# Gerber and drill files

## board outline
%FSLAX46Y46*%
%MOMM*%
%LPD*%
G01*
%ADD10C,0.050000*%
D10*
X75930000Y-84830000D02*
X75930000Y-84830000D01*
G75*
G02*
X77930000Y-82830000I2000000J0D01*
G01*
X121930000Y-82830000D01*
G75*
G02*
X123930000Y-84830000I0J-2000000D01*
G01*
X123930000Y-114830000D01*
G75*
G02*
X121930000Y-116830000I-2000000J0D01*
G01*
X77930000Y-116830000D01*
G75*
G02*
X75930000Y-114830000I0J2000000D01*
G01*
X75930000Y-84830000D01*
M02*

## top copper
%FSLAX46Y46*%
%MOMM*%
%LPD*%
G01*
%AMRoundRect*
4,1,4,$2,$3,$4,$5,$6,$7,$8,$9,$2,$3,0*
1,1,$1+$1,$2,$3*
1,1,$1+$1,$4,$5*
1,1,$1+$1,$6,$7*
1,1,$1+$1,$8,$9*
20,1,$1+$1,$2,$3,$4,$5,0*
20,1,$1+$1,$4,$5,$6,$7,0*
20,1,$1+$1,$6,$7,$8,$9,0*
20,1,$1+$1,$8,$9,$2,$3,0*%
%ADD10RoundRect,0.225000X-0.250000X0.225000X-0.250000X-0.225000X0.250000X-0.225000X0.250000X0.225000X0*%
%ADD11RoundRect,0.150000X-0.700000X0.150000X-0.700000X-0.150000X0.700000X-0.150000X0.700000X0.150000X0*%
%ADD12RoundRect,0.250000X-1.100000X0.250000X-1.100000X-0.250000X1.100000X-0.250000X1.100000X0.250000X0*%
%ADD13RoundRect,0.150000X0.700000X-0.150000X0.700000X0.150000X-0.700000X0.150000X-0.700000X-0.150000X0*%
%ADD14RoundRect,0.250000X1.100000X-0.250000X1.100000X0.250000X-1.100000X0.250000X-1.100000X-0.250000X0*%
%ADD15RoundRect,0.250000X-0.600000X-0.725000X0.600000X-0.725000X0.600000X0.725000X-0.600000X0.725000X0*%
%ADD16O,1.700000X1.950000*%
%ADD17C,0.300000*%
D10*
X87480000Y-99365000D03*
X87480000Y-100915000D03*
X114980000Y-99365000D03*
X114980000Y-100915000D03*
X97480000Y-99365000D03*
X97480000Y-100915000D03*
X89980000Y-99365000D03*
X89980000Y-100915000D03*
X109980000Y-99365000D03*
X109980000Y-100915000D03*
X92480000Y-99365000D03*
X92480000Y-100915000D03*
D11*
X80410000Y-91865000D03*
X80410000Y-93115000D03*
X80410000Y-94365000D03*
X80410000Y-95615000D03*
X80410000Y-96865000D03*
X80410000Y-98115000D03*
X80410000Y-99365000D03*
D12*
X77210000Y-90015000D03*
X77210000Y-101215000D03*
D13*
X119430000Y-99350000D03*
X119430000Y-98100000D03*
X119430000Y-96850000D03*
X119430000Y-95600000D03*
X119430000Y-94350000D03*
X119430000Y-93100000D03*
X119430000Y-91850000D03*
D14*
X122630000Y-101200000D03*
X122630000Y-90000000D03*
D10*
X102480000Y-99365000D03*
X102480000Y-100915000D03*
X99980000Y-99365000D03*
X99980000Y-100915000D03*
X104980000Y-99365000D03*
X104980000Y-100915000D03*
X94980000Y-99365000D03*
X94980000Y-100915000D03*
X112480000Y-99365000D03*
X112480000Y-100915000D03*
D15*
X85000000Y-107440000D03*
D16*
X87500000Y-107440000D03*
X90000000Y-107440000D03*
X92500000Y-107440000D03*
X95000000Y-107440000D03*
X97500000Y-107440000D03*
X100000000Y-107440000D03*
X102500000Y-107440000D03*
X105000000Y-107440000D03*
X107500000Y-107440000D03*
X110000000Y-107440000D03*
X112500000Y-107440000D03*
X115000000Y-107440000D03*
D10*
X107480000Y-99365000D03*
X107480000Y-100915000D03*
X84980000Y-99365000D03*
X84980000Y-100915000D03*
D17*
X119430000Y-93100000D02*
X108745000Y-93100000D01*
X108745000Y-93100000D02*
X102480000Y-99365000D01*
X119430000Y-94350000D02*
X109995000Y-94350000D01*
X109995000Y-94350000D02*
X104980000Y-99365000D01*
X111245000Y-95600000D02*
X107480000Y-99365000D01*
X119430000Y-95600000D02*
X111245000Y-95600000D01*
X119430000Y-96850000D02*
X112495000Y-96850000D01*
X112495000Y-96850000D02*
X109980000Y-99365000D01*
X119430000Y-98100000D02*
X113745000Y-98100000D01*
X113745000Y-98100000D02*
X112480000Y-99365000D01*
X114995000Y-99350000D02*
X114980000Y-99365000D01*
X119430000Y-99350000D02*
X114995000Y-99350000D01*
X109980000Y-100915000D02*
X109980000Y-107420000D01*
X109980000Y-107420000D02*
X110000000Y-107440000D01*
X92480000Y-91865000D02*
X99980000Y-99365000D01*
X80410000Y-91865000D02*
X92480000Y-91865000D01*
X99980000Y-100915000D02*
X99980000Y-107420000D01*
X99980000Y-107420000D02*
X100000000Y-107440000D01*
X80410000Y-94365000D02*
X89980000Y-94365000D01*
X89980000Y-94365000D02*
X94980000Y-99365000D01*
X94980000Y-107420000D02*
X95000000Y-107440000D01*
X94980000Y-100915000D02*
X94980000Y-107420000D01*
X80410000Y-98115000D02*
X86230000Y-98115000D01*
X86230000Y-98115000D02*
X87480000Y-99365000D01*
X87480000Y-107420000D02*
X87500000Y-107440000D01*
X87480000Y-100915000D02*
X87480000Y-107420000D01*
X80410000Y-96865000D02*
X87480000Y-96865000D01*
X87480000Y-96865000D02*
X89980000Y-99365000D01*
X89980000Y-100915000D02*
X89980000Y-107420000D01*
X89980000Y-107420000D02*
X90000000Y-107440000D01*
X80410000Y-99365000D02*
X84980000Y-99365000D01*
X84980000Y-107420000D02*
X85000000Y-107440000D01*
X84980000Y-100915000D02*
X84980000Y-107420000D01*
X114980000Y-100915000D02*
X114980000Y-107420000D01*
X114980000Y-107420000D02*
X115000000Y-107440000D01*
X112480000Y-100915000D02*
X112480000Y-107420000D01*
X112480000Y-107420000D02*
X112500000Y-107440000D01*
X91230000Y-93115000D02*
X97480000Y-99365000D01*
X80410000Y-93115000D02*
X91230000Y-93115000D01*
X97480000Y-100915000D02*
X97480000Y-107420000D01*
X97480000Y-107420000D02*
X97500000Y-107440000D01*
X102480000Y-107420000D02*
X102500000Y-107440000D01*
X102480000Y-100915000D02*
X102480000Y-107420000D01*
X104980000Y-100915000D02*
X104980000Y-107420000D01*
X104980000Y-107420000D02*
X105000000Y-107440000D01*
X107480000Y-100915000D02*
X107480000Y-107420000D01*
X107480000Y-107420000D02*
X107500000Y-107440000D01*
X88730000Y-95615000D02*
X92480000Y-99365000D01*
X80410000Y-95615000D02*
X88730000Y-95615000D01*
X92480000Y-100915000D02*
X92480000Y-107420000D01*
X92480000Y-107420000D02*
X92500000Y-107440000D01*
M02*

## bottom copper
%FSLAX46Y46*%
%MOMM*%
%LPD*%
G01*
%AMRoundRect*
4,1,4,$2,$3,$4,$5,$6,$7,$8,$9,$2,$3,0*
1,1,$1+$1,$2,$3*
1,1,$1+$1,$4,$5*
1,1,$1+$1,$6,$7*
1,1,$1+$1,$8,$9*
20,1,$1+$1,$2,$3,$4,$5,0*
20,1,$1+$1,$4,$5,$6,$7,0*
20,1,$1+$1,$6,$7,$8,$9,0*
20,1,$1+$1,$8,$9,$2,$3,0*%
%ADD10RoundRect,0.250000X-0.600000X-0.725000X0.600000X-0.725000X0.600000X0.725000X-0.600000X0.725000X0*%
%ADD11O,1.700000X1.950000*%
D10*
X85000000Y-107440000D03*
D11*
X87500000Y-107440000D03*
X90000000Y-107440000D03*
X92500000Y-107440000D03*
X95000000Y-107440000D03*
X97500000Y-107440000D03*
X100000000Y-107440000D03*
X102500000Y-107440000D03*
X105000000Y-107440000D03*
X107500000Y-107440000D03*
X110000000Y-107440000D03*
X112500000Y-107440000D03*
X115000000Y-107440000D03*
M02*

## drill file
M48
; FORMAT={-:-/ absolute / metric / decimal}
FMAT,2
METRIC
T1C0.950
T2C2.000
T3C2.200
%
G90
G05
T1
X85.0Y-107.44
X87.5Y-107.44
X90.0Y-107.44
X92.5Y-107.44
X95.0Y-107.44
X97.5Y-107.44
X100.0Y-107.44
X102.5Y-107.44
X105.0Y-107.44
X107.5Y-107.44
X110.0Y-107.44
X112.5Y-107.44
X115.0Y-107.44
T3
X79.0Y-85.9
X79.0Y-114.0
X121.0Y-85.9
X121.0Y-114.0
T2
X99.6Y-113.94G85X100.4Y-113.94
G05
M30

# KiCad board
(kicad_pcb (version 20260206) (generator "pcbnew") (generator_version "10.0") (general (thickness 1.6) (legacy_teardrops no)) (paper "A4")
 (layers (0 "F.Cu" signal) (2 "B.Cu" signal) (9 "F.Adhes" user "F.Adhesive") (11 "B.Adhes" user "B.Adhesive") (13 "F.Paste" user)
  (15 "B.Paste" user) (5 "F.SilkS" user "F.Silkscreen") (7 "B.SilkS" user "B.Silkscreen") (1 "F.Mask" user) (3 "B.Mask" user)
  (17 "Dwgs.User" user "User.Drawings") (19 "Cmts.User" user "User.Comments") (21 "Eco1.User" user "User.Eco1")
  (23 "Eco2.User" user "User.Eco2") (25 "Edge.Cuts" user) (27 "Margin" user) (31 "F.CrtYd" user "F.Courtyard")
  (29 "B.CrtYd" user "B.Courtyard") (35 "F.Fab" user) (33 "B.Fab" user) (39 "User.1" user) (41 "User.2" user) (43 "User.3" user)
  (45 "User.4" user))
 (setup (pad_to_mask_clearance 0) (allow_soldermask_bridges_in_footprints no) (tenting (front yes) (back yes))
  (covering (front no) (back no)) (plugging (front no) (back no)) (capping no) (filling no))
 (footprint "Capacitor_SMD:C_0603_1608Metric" (layer "F.Cu") (at 87.48 100.14 -90)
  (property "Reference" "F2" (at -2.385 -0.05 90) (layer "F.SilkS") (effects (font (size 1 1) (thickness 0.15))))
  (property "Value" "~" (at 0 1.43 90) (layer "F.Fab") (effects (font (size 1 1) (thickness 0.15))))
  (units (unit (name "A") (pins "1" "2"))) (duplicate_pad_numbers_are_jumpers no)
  (pad "1" smd roundrect (at -0.775 0 270) (size 0.9 0.95) (layers "F.Cu" "F.Mask" "F.Paste") (roundrect_rratio 0.25) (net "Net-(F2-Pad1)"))
  (pad "2" smd roundrect (at 0.775 0 270) (size 0.9 0.95) (layers "F.Cu" "F.Mask" "F.Paste") (roundrect_rratio 0.25) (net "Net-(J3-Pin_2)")))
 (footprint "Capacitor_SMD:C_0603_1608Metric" (layer "F.Cu") (at 114.98 100.14 -90)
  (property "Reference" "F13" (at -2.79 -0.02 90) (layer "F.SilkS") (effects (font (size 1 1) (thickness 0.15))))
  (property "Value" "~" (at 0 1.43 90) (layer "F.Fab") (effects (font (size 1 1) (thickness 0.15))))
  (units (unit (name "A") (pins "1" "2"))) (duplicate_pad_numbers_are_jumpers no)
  (pad "1" smd roundrect (at -0.775 0 270) (size 0.9 0.95) (layers "F.Cu" "F.Mask" "F.Paste") (roundrect_rratio 0.25) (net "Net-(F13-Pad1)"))
  (pad "2" smd roundrect (at 0.775 0 270) (size 0.9 0.95) (layers "F.Cu" "F.Mask" "F.Paste") (roundrect_rratio 0.25) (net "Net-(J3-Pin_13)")))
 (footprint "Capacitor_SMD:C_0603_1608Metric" (layer "F.Cu") (at 97.48 100.14 -90)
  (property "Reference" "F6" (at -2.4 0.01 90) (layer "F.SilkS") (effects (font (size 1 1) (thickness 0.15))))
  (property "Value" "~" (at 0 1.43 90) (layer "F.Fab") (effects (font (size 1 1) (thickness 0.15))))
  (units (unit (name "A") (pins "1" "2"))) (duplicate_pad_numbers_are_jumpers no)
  (pad "1" smd roundrect (at -0.775 0 270) (size 0.9 0.95) (layers "F.Cu" "F.Mask" "F.Paste") (roundrect_rratio 0.25) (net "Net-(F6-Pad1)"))
  (pad "2" smd roundrect (at 0.775 0 270) (size 0.9 0.95) (layers "F.Cu" "F.Mask" "F.Paste") (roundrect_rratio 0.25) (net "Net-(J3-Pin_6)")))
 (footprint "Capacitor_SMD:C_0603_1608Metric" (layer "F.Cu") (at 89.98 100.14 -90)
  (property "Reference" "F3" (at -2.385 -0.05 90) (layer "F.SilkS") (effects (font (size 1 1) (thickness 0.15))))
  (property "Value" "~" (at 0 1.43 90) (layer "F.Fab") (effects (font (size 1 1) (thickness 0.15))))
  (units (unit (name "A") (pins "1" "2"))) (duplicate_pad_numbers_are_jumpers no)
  (pad "1" smd roundrect (at -0.775 0 270) (size 0.9 0.95) (layers "F.Cu" "F.Mask" "F.Paste") (roundrect_rratio 0.25) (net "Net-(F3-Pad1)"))
  (pad "2" smd roundrect (at 0.775 0 270) (size 0.9 0.95) (layers "F.Cu" "F.Mask" "F.Paste") (roundrect_rratio 0.25) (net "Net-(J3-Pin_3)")))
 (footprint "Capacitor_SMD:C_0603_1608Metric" (layer "F.Cu") (at 109.98 100.14 -90)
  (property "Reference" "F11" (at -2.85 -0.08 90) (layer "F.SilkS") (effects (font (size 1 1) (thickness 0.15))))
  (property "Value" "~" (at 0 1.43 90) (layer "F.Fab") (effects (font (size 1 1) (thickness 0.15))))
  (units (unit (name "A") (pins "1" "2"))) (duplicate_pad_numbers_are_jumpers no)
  (pad "1" smd roundrect (at -0.775 0 270) (size 0.9 0.95) (layers "F.Cu" "F.Mask" "F.Paste") (roundrect_rratio 0.25) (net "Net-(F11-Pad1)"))
  (pad "2" smd roundrect (at 0.775 0 270) (size 0.9 0.95) (layers "F.Cu" "F.Mask" "F.Paste") (roundrect_rratio 0.25) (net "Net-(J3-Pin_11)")))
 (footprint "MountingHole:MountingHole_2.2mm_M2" (layer "F.Cu") (at 121 114)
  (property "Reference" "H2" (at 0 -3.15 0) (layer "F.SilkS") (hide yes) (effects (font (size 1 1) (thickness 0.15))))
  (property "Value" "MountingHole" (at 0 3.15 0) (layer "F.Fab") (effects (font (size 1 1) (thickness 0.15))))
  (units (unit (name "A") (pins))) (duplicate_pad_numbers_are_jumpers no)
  (pad "" np_thru_hole circle (at 0 0) (size 2.2 2.2) (drill 2.2) (layers "*.Cu" "*.Mask")))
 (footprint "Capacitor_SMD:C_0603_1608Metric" (layer "F.Cu") (at 92.48 100.14 -90)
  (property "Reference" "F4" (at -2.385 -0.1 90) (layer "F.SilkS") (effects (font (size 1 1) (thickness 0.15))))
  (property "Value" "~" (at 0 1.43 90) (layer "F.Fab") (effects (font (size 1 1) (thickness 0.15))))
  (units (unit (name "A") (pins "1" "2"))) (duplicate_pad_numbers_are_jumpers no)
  (pad "1" smd roundrect (at -0.775 0 270) (size 0.9 0.95) (layers "F.Cu" "F.Mask" "F.Paste") (roundrect_rratio 0.25) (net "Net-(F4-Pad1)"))
  (pad "2" smd roundrect (at 0.775 0 270) (size 0.9 0.95) (layers "F.Cu" "F.Mask" "F.Paste") (roundrect_rratio 0.25) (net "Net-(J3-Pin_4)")))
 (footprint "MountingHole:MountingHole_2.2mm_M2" (layer "F.Cu") (at 121 85.9)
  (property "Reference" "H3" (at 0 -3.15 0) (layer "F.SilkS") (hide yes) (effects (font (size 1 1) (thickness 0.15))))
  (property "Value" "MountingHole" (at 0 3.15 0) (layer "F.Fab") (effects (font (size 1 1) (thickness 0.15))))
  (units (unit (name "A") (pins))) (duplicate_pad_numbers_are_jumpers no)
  (pad "" np_thru_hole circle (at 0 0) (size 2.2 2.2) (drill 2.2) (layers "*.Cu" "*.Mask")))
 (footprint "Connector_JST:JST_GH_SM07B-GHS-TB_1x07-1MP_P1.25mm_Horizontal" (layer "F.Cu") (at 78.56 95.615 -90)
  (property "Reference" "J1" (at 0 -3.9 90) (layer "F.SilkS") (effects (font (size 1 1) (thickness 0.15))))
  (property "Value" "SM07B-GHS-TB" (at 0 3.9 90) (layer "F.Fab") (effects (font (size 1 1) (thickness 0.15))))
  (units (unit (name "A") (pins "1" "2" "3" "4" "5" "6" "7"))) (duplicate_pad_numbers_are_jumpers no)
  (pad "1" smd roundrect (at -3.75 -1.85 270) (size 0.6 1.7) (layers "F.Cu" "F.Mask" "F.Paste") (roundrect_rratio 0.25)
   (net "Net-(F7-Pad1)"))
  (pad "2" smd roundrect (at -2.5 -1.85 270) (size 0.6 1.7) (layers "F.Cu" "F.Mask" "F.Paste") (roundrect_rratio 0.25) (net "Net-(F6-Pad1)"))
  (pad "3" smd roundrect (at -1.25 -1.85 270) (size 0.6 1.7) (layers "F.Cu" "F.Mask" "F.Paste") (roundrect_rratio 0.25)
   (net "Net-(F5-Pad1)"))
  (pad "4" smd roundrect (at 0 -1.85 270) (size 0.6 1.7) (layers "F.Cu" "F.Mask" "F.Paste") (roundrect_rratio 0.25) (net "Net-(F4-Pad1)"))
  (pad "5" smd roundrect (at 1.25 -1.85 270) (size 0.6 1.7) (layers "F.Cu" "F.Mask" "F.Paste") (roundrect_rratio 0.25) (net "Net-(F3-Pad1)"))
  (pad "6" smd roundrect (at 2.5 -1.85 270) (size 0.6 1.7) (layers "F.Cu" "F.Mask" "F.Paste") (roundrect_rratio 0.25) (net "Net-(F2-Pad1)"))
  (pad "7" smd roundrect (at 3.75 -1.85 270) (size 0.6 1.7) (layers "F.Cu" "F.Mask" "F.Paste") (roundrect_rratio 0.25) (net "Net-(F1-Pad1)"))
  (pad "MP" smd roundrect (at -5.6 1.35 270) (size 1 2.7) (layers "F.Cu" "F.Mask" "F.Paste") (roundrect_rratio 0.25))
  (pad "MP" smd roundrect (at 5.6 1.35 270) (size 1 2.7) (layers "F.Cu" "F.Mask" "F.Paste") (roundrect_rratio 0.25)))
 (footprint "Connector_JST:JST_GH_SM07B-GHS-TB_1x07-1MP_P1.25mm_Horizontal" (layer "F.Cu") (at 121.28 95.6 90)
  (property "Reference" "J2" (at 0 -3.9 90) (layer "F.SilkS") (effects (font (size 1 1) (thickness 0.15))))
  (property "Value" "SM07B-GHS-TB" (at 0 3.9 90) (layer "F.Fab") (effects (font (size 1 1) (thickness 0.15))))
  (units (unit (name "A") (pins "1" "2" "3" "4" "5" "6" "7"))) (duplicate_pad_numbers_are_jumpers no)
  (pad "1" smd roundrect (at -3.75 -1.85 90) (size 0.6 1.7) (layers "F.Cu" "F.Mask" "F.Paste") (roundrect_rratio 0.25)
   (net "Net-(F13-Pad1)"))
  (pad "2" smd roundrect (at -2.5 -1.85 90) (size 0.6 1.7) (layers "F.Cu" "F.Mask" "F.Paste") (roundrect_rratio 0.25) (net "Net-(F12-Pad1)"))
  (pad "3" smd roundrect (at -1.25 -1.85 90) (size 0.6 1.7) (layers "F.Cu" "F.Mask" "F.Paste") (roundrect_rratio 0.25)
   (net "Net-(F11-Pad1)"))
  (pad "4" smd roundrect (at 0 -1.85 90) (size 0.6 1.7) (layers "F.Cu" "F.Mask" "F.Paste") (roundrect_rratio 0.25) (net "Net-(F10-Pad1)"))
  (pad "5" smd roundrect (at 1.25 -1.85 90) (size 0.6 1.7) (layers "F.Cu" "F.Mask" "F.Paste") (roundrect_rratio 0.25) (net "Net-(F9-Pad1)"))
  (pad "6" smd roundrect (at 2.5 -1.85 90) (size 0.6 1.7) (layers "F.Cu" "F.Mask" "F.Paste") (roundrect_rratio 0.25) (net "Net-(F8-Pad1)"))
  (pad "7" smd roundrect (at 3.75 -1.85 90) (size 0.6 1.7) (layers "F.Cu" "F.Mask" "F.Paste") (roundrect_rratio 0.25)
   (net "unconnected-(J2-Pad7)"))
  (pad "MP" smd roundrect (at -5.6 1.35 90) (size 1 2.7) (layers "F.Cu" "F.Mask" "F.Paste") (roundrect_rratio 0.25))
  (pad "MP" smd roundrect (at 5.6 1.35 90) (size 1 2.7) (layers "F.Cu" "F.Mask" "F.Paste") (roundrect_rratio 0.25)))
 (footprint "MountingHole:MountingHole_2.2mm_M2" (layer "F.Cu") (at 79 85.9)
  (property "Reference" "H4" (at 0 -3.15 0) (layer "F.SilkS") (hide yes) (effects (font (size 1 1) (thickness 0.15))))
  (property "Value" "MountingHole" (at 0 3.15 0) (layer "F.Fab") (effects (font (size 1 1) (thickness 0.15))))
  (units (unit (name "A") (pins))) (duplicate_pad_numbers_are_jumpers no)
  (pad "" np_thru_hole circle (at 0 0) (size 2.2 2.2) (drill 2.2) (layers "*.Cu" "*.Mask")))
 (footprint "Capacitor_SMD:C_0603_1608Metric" (layer "F.Cu") (at 102.48 100.14 -90)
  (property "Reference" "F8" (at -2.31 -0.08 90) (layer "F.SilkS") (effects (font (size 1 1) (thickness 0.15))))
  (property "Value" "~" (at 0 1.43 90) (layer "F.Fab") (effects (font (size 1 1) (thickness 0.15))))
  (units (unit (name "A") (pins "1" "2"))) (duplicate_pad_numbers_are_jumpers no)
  (pad "1" smd roundrect (at -0.775 0 270) (size 0.9 0.95) (layers "F.Cu" "F.Mask" "F.Paste") (roundrect_rratio 0.25) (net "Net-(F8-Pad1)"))
  (pad "2" smd roundrect (at 0.775 0 270) (size 0.9 0.95) (layers "F.Cu" "F.Mask" "F.Paste") (roundrect_rratio 0.25) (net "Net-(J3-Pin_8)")))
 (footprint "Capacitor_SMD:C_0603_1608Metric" (layer "F.Cu") (at 99.98 100.14 -90)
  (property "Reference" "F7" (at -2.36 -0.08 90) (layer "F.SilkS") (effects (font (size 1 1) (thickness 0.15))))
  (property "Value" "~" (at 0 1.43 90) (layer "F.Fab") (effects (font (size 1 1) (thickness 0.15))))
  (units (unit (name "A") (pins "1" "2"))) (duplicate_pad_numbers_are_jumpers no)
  (pad "1" smd roundrect (at -0.775 0 270) (size 0.9 0.95) (layers "F.Cu" "F.Mask" "F.Paste") (roundrect_rratio 0.25) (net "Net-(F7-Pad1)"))
  (pad "2" smd roundrect (at 0.775 0 270) (size 0.9 0.95) (layers "F.Cu" "F.Mask" "F.Paste") (roundrect_rratio 0.25) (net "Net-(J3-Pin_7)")))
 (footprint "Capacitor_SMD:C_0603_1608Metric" (layer "F.Cu") (at 104.98 100.14 -90)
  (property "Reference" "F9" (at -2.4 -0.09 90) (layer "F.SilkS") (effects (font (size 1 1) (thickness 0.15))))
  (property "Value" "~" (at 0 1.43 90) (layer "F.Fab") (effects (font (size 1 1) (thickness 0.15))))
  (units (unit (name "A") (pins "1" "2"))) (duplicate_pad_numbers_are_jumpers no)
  (pad "1" smd roundrect (at -0.775 0 270) (size 0.9 0.95) (layers "F.Cu" "F.Mask" "F.Paste") (roundrect_rratio 0.25) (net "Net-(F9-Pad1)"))
  (pad "2" smd roundrect (at 0.775 0 270) (size 0.9 0.95) (layers "F.Cu" "F.Mask" "F.Paste") (roundrect_rratio 0.25) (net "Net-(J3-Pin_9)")))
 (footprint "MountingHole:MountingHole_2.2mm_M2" (layer "F.Cu") (at 79 114)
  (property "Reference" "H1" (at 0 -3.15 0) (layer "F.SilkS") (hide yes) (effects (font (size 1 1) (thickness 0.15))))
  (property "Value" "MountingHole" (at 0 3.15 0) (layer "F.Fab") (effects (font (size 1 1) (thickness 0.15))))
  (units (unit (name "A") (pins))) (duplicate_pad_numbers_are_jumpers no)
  (pad "" np_thru_hole circle (at 0 0) (size 2.2 2.2) (drill 2.2) (layers "*.Cu" "*.Mask")))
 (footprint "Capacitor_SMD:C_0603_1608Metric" (layer "F.Cu") (at 94.98 100.14 -90)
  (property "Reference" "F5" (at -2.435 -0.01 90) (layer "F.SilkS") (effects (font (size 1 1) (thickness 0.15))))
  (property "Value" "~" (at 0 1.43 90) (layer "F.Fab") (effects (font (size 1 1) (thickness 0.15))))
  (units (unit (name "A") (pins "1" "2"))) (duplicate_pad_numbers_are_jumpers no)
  (pad "1" smd roundrect (at -0.775 0 270) (size 0.9 0.95) (layers "F.Cu" "F.Mask" "F.Paste") (roundrect_rratio 0.25) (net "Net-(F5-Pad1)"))
  (pad "2" smd roundrect (at 0.775 0 270) (size 0.9 0.95) (layers "F.Cu" "F.Mask" "F.Paste") (roundrect_rratio 0.25) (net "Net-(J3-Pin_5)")))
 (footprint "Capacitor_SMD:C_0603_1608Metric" (layer "F.Cu") (at 112.48 100.14 -90)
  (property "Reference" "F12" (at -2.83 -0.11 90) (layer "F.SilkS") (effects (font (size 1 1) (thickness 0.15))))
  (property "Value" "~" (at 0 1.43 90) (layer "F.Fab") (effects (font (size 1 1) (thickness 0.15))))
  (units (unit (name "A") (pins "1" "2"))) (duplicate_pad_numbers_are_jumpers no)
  (pad "1" smd roundrect (at -0.775 0 270) (size 0.9 0.95) (layers "F.Cu" "F.Mask" "F.Paste") (roundrect_rratio 0.25) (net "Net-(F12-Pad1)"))
  (pad "2" smd roundrect (at 0.775 0 270) (size 0.9 0.95) (layers "F.Cu" "F.Mask" "F.Paste") (roundrect_rratio 0.25) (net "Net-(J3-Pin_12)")))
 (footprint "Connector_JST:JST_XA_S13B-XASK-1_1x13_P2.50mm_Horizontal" (layer "F.Cu") (at 85 107.44)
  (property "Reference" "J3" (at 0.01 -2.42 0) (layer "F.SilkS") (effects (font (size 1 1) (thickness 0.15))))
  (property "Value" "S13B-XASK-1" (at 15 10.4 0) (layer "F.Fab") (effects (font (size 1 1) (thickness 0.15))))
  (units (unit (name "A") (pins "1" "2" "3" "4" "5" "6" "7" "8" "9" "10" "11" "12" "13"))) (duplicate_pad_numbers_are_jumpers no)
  (pad "" np_thru_hole oval (at 15 6.5) (size 2.8 2) (drill oval 2.8 2) (layers "*.Cu" "*.Mask"))
  (pad "1" thru_hole roundrect (at 0 0) (size 1.7 1.95) (drill 0.95) (layers "*.Cu" "*.Mask") (remove_unused_layers no)
   (roundrect_rratio 0.147059) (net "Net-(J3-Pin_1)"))
  (pad "2" thru_hole oval (at 2.5 0) (size 1.7 1.95) (drill 0.95) (layers "*.Cu" "*.Mask") (remove_unused_layers no) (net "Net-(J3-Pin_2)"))
  (pad "3" thru_hole oval (at 5 0) (size 1.7 1.95) (drill 0.95) (layers "*.Cu" "*.Mask") (remove_unused_layers no) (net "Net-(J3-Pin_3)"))
  (pad "4" thru_hole oval (at 7.5 0) (size 1.7 1.95) (drill 0.95) (layers "*.Cu" "*.Mask") (remove_unused_layers no) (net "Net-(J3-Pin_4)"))
  (pad "5" thru_hole oval (at 10 0) (size 1.7 1.95) (drill 0.95) (layers "*.Cu" "*.Mask") (remove_unused_layers no) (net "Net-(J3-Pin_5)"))
  (pad "6" thru_hole oval (at 12.5 0) (size 1.7 1.95) (drill 0.95) (layers "*.Cu" "*.Mask") (remove_unused_layers no) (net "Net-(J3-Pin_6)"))
  (pad "7" thru_hole oval (at 15 0) (size 1.7 1.95) (drill 0.95) (layers "*.Cu" "*.Mask") (remove_unused_layers no) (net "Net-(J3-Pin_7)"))
  (pad "8" thru_hole oval (at 17.5 0) (size 1.7 1.95) (drill 0.95) (layers "*.Cu" "*.Mask") (remove_unused_layers no) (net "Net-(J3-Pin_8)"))
  (pad "9" thru_hole oval (at 20 0) (size 1.7 1.95) (drill 0.95) (layers "*.Cu" "*.Mask") (remove_unused_layers no) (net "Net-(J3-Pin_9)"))
  (pad "10" thru_hole oval (at 22.5 0) (size 1.7 1.95) (drill 0.95) (layers "*.Cu" "*.Mask") (remove_unused_layers no)
   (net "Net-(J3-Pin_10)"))
  (pad "11" thru_hole oval (at 25 0) (size 1.7 1.95) (drill 0.95) (layers "*.Cu" "*.Mask") (remove_unused_layers no) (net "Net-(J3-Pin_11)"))
  (pad "12" thru_hole oval (at 27.5 0) (size 1.7 1.95) (drill 0.95) (layers "*.Cu" "*.Mask") (remove_unused_layers no)
   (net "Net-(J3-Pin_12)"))
  (pad "13" thru_hole oval (at 30 0) (size 1.7 1.95) (drill 0.95) (layers "*.Cu" "*.Mask") (remove_unused_layers no) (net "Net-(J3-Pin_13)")))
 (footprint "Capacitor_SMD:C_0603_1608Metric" (layer "F.Cu") (at 107.48 100.14 -90)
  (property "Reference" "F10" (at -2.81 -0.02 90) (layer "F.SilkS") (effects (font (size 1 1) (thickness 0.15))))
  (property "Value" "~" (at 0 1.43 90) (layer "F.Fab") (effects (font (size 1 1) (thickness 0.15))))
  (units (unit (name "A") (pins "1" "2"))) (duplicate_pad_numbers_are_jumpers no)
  (pad "1" smd roundrect (at -0.775 0 270) (size 0.9 0.95) (layers "F.Cu" "F.Mask" "F.Paste") (roundrect_rratio 0.25) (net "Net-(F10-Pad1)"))
  (pad "2" smd roundrect (at 0.775 0 270) (size 0.9 0.95) (layers "F.Cu" "F.Mask" "F.Paste") (roundrect_rratio 0.25) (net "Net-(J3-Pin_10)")))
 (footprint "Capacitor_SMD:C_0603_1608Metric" (layer "F.Cu") (at 84.98 100.14 -90)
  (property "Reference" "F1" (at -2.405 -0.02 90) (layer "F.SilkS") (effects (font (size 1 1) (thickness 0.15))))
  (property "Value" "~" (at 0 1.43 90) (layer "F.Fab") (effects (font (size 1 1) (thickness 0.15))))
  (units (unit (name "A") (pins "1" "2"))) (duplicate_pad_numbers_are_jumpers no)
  (pad "1" smd roundrect (at -0.775 0 270) (size 0.9 0.95) (layers "F.Cu" "F.Mask" "F.Paste") (roundrect_rratio 0.25) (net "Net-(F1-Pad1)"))
  (pad "2" smd roundrect (at 0.775 0 270) (size 0.9 0.95) (layers "F.Cu" "F.Mask" "F.Paste") (roundrect_rratio 0.25) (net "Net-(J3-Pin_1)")))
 (gr_rect (start 75.93 82.83) (end 123.93 116.83) (radius 2) (stroke (width 0.05) (type solid)) (fill no) (layer "Edge.Cuts"))
 (segment (start 119.43 93.1) (end 108.745 93.1) (width 0.3) (layer "F.Cu") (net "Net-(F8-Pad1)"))
 (segment (start 108.745 93.1) (end 102.48 99.365) (width 0.3) (layer "F.Cu") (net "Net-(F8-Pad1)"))
 (segment (start 119.43 94.35) (end 109.995 94.35) (width 0.3) (layer "F.Cu") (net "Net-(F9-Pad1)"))
 (segment (start 109.995 94.35) (end 104.98 99.365) (width 0.3) (layer "F.Cu") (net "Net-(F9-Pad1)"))
 (segment (start 111.245 95.6) (end 107.48 99.365) (width 0.3) (layer "F.Cu") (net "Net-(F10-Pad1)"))
 (segment (start 119.43 95.6) (end 111.245 95.6) (width 0.3) (layer "F.Cu") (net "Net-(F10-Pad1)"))
 (segment (start 119.43 96.85) (end 112.495 96.85) (width 0.3) (layer "F.Cu") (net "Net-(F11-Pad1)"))
 (segment (start 112.495 96.85) (end 109.98 99.365) (width 0.3) (layer "F.Cu") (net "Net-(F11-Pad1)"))
 (segment (start 119.43 98.1) (end 113.745 98.1) (width 0.3) (layer "F.Cu") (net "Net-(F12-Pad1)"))
 (segment (start 113.745 98.1) (end 112.48 99.365) (width 0.3) (layer "F.Cu") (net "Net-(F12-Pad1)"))
 (segment (start 114.995 99.35) (end 114.98 99.365) (width 0.3) (layer "F.Cu") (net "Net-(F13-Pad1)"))
 (segment (start 119.43 99.35) (end 114.995 99.35) (width 0.3) (layer "F.Cu") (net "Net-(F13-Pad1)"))
 (segment (start 109.98 100.915) (end 109.98 107.42) (width 0.3) (layer "F.Cu") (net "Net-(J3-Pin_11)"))
 (segment (start 109.98 107.42) (end 110 107.44) (width 0.3) (layer "F.Cu") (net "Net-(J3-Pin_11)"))
 (segment (start 92.48 91.865) (end 99.98 99.365) (width 0.3) (layer "F.Cu") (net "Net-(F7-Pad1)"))
 (segment (start 80.41 91.865) (end 92.48 91.865) (width 0.3) (layer "F.Cu") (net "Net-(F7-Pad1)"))
 (segment (start 99.98 100.915) (end 99.98 107.42) (width 0.3) (layer "F.Cu") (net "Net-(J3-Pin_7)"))
 (segment (start 99.98 107.42) (end 100 107.44) (width 0.3) (layer "F.Cu") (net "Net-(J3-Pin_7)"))
 (segment (start 80.41 94.365) (end 89.98 94.365) (width 0.3) (layer "F.Cu") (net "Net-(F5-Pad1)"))
 (segment (start 89.98 94.365) (end 94.98 99.365) (width 0.3) (layer "F.Cu") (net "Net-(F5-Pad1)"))
 (segment (start 94.98 107.42) (end 95 107.44) (width 0.3) (layer "F.Cu") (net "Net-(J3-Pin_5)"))
 (segment (start 94.98 100.915) (end 94.98 107.42) (width 0.3) (layer "F.Cu") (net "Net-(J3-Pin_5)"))
 (segment (start 80.41 98.115) (end 86.23 98.115) (width 0.3) (layer "F.Cu") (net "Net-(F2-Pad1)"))
 (segment (start 86.23 98.115) (end 87.48 99.365) (width 0.3) (layer "F.Cu") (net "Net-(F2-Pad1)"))
 (segment (start 87.48 107.42) (end 87.5 107.44) (width 0.3) (layer "F.Cu") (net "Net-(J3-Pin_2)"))
 (segment (start 87.48 100.915) (end 87.48 107.42) (width 0.3) (layer "F.Cu") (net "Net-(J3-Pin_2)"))
 (segment (start 80.41 96.865) (end 87.48 96.865) (width 0.3) (layer "F.Cu") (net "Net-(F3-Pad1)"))
 (segment (start 87.48 96.865) (end 89.98 99.365) (width 0.3) (layer "F.Cu") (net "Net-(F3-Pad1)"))
 (segment (start 89.98 100.915) (end 89.98 107.42) (width 0.3) (layer "F.Cu") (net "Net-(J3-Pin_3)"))
 (segment (start 89.98 107.42) (end 90 107.44) (width 0.3) (layer "F.Cu") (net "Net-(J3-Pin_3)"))
 (segment (start 80.41 99.365) (end 84.98 99.365) (width 0.3) (layer "F.Cu") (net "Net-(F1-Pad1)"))
 (segment (start 84.98 107.42) (end 85 107.44) (width 0.3) (layer "F.Cu") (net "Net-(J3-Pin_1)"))
 (segment (start 84.98 100.915) (end 84.98 107.42) (width 0.3) (layer "F.Cu") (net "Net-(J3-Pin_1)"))
 (segment (start 114.98 100.915) (end 114.98 107.42) (width 0.3) (layer "F.Cu") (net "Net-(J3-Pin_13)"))
 (segment (start 114.98 107.42) (end 115 107.44) (width 0.3) (layer "F.Cu") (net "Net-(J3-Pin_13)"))
 (segment (start 112.48 100.915) (end 112.48 107.42) (width 0.3) (layer "F.Cu") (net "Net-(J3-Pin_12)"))
 (segment (start 112.48 107.42) (end 112.5 107.44) (width 0.3) (layer "F.Cu") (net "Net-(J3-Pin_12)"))
 (segment (start 91.23 93.115) (end 97.48 99.365) (width 0.3) (layer "F.Cu") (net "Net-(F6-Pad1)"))
 (segment (start 80.41 93.115) (end 91.23 93.115) (width 0.3) (layer "F.Cu") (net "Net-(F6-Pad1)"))
 (segment (start 97.48 100.915) (end 97.48 107.42) (width 0.3) (layer "F.Cu") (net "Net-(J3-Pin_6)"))
 (segment (start 97.48 107.42) (end 97.5 107.44) (width 0.3) (layer "F.Cu") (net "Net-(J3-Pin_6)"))
 (segment (start 102.48 107.42) (end 102.5 107.44) (width 0.3) (layer "F.Cu") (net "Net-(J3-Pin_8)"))
 (segment (start 102.48 100.915) (end 102.48 107.42) (width 0.3) (layer "F.Cu") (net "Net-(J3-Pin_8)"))
 (segment (start 104.98 100.915) (end 104.98 107.42) (width 0.3) (layer "F.Cu") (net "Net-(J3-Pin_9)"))
 (segment (start 104.98 107.42) (end 105 107.44) (width 0.3) (layer "F.Cu") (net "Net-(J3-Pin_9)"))
 (segment (start 107.48 100.915) (end 107.48 107.42) (width 0.3) (layer "F.Cu") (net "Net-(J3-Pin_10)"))
 (segment (start 107.48 107.42) (end 107.5 107.44) (width 0.3) (layer "F.Cu") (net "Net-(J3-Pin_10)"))
 (segment (start 88.73 95.615) (end 92.48 99.365) (width 0.3) (layer "F.Cu") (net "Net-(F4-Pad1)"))
 (segment (start 80.41 95.615) (end 88.73 95.615) (width 0.3) (layer "F.Cu") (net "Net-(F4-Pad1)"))
 (segment (start 92.48 100.915) (end 92.48 107.42) (width 0.3) (layer "F.Cu") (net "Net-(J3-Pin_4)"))
 (segment (start 92.48 107.42) (end 92.5 107.44) (width 0.3) (layer "F.Cu") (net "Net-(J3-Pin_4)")))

